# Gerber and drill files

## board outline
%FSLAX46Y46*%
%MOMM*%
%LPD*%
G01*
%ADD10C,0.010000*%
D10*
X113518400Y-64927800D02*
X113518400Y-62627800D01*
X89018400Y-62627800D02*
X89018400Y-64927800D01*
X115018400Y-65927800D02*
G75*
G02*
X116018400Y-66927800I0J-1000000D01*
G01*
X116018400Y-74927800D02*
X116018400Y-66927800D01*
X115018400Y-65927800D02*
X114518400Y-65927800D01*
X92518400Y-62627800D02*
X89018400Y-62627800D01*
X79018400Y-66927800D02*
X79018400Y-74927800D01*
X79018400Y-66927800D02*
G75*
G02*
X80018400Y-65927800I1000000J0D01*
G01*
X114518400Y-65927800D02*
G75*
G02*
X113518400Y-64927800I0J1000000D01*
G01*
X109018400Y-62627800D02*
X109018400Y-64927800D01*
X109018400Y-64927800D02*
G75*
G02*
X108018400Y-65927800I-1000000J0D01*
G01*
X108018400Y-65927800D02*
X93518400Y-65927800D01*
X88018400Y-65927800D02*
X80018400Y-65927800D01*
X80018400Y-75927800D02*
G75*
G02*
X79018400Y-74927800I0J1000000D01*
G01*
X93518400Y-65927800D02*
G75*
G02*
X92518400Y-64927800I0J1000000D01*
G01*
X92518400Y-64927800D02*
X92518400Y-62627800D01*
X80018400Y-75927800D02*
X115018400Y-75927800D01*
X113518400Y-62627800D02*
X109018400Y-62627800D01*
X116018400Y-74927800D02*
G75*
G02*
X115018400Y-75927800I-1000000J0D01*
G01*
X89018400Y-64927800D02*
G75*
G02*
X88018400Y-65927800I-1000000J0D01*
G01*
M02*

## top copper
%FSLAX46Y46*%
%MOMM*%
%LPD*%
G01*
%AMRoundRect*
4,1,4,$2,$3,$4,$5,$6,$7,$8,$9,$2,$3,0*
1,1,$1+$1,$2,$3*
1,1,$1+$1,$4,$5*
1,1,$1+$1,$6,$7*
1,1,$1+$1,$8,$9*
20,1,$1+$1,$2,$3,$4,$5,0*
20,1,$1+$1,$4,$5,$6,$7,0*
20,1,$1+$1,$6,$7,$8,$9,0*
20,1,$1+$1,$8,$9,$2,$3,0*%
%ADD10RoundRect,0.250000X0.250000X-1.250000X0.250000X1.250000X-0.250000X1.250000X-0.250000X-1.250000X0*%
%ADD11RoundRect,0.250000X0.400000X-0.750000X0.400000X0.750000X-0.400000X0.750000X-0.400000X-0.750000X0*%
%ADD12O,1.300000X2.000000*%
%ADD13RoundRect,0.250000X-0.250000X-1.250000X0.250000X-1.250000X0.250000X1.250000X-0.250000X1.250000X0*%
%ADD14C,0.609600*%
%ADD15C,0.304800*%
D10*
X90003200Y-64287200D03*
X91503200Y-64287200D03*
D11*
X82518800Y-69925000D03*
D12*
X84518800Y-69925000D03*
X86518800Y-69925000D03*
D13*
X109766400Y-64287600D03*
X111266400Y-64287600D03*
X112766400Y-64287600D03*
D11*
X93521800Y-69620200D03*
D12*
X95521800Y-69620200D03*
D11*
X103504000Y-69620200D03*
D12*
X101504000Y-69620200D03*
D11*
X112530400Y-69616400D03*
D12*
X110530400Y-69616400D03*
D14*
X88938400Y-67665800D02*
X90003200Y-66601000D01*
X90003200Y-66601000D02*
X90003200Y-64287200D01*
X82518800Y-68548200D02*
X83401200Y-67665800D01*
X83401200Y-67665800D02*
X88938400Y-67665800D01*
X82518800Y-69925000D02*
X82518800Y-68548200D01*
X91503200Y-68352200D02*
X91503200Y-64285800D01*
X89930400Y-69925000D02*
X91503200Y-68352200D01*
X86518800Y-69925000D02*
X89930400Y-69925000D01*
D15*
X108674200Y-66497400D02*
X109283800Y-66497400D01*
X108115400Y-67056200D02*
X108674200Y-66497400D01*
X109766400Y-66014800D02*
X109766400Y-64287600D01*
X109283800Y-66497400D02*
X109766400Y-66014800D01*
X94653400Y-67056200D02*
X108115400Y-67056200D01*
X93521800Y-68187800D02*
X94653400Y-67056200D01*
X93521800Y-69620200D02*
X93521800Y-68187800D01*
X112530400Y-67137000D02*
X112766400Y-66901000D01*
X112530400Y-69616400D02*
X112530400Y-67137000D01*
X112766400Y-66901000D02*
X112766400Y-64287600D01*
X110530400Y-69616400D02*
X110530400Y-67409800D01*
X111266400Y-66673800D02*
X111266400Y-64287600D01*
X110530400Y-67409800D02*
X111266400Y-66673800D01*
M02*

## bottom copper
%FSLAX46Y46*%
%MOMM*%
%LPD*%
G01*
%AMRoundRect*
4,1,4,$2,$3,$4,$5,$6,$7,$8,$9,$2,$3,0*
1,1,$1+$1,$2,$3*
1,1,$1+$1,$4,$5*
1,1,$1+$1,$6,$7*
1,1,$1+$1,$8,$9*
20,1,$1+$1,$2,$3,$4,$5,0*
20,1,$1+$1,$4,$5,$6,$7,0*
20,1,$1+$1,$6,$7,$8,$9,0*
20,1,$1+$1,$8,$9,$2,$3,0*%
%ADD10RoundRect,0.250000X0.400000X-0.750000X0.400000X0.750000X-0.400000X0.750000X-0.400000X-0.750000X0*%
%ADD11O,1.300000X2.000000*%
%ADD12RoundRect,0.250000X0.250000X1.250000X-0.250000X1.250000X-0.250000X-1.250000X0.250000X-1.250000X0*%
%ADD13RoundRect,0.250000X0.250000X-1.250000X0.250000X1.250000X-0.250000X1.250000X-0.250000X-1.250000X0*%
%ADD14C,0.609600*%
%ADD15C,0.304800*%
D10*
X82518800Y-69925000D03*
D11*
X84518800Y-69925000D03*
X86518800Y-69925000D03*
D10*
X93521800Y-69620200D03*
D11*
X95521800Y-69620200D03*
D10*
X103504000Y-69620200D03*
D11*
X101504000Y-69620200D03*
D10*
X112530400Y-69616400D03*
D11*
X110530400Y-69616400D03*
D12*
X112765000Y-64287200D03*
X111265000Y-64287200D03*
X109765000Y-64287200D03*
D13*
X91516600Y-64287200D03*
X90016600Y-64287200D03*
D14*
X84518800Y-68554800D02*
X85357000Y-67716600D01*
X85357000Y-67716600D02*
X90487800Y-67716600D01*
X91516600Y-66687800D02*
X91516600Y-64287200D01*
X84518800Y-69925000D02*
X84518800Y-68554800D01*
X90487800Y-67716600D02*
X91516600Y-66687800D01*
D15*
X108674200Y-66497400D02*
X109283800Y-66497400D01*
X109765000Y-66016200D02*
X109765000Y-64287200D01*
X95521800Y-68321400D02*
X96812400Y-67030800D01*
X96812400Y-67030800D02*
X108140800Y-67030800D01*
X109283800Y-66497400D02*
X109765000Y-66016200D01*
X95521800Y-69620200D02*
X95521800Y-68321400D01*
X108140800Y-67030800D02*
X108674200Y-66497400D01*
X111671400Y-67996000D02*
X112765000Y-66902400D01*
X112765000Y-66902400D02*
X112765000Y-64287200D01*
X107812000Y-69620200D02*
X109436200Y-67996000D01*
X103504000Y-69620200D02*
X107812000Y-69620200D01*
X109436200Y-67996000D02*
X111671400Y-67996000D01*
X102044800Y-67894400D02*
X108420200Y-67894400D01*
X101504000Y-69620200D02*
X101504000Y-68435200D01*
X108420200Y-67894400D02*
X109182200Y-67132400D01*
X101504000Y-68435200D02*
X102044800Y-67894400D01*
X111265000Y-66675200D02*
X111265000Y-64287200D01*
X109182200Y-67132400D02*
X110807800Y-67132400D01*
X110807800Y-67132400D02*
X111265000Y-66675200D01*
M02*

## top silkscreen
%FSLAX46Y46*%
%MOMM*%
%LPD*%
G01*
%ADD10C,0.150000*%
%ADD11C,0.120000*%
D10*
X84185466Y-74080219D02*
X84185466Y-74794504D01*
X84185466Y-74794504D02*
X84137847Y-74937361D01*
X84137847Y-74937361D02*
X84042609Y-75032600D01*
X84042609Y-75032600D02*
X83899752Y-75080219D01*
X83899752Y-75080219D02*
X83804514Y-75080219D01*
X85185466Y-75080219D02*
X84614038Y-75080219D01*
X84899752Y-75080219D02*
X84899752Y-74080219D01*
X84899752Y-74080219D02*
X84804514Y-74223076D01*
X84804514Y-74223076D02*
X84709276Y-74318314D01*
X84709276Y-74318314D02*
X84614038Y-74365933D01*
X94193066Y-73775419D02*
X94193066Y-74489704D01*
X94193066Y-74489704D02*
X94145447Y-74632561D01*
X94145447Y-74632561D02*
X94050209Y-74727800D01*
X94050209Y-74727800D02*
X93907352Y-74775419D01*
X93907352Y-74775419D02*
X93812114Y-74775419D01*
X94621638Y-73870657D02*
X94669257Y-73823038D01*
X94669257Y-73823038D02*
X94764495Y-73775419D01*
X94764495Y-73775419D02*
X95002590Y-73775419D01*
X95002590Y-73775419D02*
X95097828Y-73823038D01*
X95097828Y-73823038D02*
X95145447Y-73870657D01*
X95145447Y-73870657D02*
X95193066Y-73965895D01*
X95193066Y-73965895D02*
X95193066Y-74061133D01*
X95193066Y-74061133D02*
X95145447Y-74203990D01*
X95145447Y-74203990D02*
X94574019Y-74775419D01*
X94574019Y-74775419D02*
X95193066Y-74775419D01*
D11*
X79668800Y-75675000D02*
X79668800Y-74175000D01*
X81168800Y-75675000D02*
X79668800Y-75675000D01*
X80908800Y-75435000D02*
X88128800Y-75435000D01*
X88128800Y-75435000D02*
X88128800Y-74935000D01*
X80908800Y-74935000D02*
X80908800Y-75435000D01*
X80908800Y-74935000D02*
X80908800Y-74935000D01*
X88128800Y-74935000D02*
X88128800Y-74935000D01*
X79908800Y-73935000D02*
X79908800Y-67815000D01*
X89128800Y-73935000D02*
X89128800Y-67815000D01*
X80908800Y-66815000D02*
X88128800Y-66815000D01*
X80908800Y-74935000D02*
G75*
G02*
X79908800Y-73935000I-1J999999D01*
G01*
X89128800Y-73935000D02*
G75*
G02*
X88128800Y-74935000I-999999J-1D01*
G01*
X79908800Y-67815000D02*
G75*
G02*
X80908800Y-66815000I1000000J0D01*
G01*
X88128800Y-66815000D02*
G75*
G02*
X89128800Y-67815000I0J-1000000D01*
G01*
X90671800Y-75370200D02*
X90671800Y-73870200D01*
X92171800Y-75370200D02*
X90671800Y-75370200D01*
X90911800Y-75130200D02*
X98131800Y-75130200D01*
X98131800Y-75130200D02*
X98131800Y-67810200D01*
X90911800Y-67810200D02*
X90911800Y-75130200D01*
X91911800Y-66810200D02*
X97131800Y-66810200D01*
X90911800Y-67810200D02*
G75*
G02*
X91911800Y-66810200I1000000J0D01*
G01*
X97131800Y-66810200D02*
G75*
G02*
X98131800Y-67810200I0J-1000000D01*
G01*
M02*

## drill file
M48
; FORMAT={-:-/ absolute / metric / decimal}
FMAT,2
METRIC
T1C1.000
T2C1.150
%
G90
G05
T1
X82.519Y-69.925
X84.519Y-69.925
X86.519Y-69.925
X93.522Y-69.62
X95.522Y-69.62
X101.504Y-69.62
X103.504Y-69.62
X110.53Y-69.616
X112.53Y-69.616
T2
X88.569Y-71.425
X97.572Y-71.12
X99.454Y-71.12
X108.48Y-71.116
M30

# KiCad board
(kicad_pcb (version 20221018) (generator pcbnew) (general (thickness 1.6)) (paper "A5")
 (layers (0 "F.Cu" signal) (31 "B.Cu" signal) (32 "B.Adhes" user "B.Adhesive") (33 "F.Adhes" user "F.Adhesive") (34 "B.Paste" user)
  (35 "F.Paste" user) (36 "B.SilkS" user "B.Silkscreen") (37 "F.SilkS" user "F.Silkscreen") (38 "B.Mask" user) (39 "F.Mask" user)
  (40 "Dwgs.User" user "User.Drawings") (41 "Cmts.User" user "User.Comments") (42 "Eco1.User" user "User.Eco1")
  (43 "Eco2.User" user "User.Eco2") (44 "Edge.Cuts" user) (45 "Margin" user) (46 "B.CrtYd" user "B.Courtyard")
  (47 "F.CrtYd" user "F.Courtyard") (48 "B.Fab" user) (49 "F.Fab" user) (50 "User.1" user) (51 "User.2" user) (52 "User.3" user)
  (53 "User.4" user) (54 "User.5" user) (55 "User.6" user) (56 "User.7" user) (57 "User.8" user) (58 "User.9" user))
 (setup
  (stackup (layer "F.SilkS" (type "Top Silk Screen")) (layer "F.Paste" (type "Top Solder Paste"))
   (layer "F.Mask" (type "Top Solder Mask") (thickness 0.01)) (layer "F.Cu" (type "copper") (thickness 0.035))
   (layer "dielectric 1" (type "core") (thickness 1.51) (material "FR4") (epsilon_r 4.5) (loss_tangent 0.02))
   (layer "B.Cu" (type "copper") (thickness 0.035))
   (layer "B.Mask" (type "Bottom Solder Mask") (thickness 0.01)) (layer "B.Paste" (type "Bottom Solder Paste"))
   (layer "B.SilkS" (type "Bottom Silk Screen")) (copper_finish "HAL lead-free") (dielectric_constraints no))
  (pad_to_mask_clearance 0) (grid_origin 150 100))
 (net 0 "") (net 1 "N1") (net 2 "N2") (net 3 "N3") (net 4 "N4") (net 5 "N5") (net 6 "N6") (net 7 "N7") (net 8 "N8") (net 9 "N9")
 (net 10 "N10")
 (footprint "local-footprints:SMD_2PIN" (layer "F.Cu") (at 90.7532 63.7872)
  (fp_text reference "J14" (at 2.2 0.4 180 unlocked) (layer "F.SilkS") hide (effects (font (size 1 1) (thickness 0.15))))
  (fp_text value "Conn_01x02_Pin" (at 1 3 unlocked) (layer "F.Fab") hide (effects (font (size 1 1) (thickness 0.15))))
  (pad "1" smd roundrect (at -0.75 0.5 90) (size 3 1) (layers "F.Cu" "F.Paste" "F.Mask") (roundrect_rratio 0.25) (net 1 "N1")
   (thermal_bridge_angle 45))
  (pad "2" smd roundrect (at 0.75 0.5 90) (size 3 1) (layers "F.Cu" "F.Paste" "F.Mask") (roundrect_rratio 0.25) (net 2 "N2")
   (thermal_bridge_angle 45)))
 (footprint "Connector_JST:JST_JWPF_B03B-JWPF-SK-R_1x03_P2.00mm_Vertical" (layer "F.Cu") (at 82.5188 69.925 90)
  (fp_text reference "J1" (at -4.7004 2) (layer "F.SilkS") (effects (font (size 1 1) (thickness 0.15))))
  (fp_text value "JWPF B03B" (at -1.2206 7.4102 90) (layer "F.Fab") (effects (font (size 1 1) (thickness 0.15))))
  (fp_line (start -5.75 -2.85) (end -4.25 -2.85) (stroke (width 0.12) (type solid)) (layer "F.SilkS"))
  (fp_line (start -5.75 -1.35) (end -5.75 -2.85) (stroke (width 0.12) (type solid)) (layer "F.SilkS"))
  (fp_line (start -5.51 -1.61) (end -5.51 5.61) (stroke (width 0.12) (type solid)) (layer "F.SilkS"))
  (fp_line (start -5.51 5.61) (end -5.01 5.61) (stroke (width 0.12) (type solid)) (layer "F.SilkS"))
  (fp_line (start -5.01 -1.61) (end -5.51 -1.61) (stroke (width 0.12) (type solid)) (layer "F.SilkS"))
  (fp_line (start -5.01 -1.61) (end -5.01 -1.61) (stroke (width 0.12) (type solid)) (layer "F.SilkS"))
  (fp_line (start -5.01 5.61) (end -5.01 5.61) (stroke (width 0.12) (type solid)) (layer "F.SilkS"))
  (fp_line (start -4.01 -2.61) (end 2.11 -2.61) (stroke (width 0.12) (type solid)) (layer "F.SilkS"))
  (fp_line (start -4.01 6.61) (end 2.11 6.61) (stroke (width 0.12) (type solid)) (layer "F.SilkS"))
  (fp_line (start 3.11 -1.61) (end 3.11 5.61) (stroke (width 0.12) (type solid)) (layer "F.SilkS"))
  (fp_arc (start -5.01 -1.61) (mid -4.717107 -2.317107) (end -4.01 -2.61) (stroke (width 0.12) (type solid)) (layer "F.SilkS"))
  (fp_arc (start -4.01 6.61) (mid -4.717107 6.317107) (end -5.01 5.61) (stroke (width 0.12) (type solid)) (layer "F.SilkS"))
  (fp_arc (start 2.11 -2.61) (mid 2.817107 -2.317107) (end 3.11 -1.61) (stroke (width 0.12) (type solid)) (layer "F.SilkS"))
  (fp_arc (start 3.11 5.61) (mid 2.817107 6.317107) (end 2.11 6.61) (stroke (width 0.12) (type solid)) (layer "F.SilkS"))
  (pad "" np_thru_hole circle (at -1.5 6.05 90) (size 1.15 1.15) (drill 1.15) (layers "*.Cu" "*.Mask"))
  (pad "1" thru_hole roundrect (at 0 0 90) (size 2 1.3) (drill 1) (layers "*.Cu" "*.Mask") (roundrect_rratio 0.1923076923) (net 1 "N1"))
  (pad "2" thru_hole oval (at 0 2 90) (size 2 1.3) (drill 1) (layers "*.Cu" "*.Mask") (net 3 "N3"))
  (pad "3" thru_hole oval (at 0 4 90) (size 2 1.3) (drill 1) (layers "*.Cu" "*.Mask") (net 2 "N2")))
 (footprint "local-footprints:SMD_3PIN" (layer "F.Cu") (at 111.2664 63.7876)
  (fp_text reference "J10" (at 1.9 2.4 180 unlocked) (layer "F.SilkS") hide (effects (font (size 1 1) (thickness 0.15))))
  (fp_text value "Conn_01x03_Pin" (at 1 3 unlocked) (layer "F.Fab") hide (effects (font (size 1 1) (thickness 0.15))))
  (pad "1" smd roundrect (at -1.5 0.5) (size 1 3) (layers "F.Cu" "F.Paste" "F.Mask") (roundrect_rratio 0.25) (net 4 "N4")
   (thermal_bridge_angle 45))
  (pad "2" smd roundrect (at 0 0.5) (size 1 3) (layers "F.Cu" "F.Paste" "F.Mask") (roundrect_rratio 0.25) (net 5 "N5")
   (thermal_bridge_angle 45))
  (pad "3" smd roundrect (at 1.5 0.5) (size 1 3) (layers "F.Cu" "F.Paste" "F.Mask") (roundrect_rratio 0.25) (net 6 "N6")
   (thermal_bridge_angle 45)))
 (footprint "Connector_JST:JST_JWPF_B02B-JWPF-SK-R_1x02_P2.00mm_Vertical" (layer "F.Cu") (at 93.5218 69.6202 90)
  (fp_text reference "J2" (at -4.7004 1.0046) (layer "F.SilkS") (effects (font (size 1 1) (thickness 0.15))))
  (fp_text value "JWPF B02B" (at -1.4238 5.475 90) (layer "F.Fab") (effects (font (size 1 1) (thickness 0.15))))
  (fp_line (start -5.75 -2.85) (end -4.25 -2.85) (stroke (width 0.12) (type solid)) (layer "F.SilkS"))
  (fp_line (start -5.75 -1.35) (end -5.75 -2.85) (stroke (width 0.12) (type solid)) (layer "F.SilkS"))
  (fp_line (start -5.51 -2.61) (end -5.51 4.61) (stroke (width 0.12) (type solid)) (layer "F.SilkS"))
  (fp_line (start -5.51 4.61) (end 1.81 4.61) (stroke (width 0.12) (type solid)) (layer "F.SilkS"))
  (fp_line (start 1.81 -2.61) (end -5.51 -2.61) (stroke (width 0.12) (type solid)) (layer "F.SilkS"))
  (fp_line (start 2.81 -1.61) (end 2.81 3.61) (stroke (width 0.12) (type solid)) (layer "F.SilkS"))
  (fp_arc (start 1.81 -2.61) (mid 2.517107 -2.317107) (end 2.81 -1.61) (stroke (width 0.12) (type solid)) (layer "F.SilkS"))
  (fp_arc (start 2.81 3.61) (mid 2.517107 4.317107) (end 1.81 4.61) (stroke (width 0.12) (type solid)) (layer "F.SilkS"))
  (pad "" np_thru_hole circle (at -1.5 4.05 90) (size 1.15 1.15) (drill 1.15) (layers "*.Cu" "*.Mask"))
  (pad "1" thru_hole roundrect (at 0 0 90) (size 2 1.3) (drill 1) (layers "*.Cu" "*.Mask") (roundrect_rratio 0.1923076923) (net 4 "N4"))
  (pad "2" thru_hole oval (at 0 2 90) (size 2 1.3) (drill 1) (layers "*.Cu" "*.Mask") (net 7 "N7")))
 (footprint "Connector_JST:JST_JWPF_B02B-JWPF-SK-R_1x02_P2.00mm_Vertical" (layer "B.Cu") (at 103.504 69.6202 90)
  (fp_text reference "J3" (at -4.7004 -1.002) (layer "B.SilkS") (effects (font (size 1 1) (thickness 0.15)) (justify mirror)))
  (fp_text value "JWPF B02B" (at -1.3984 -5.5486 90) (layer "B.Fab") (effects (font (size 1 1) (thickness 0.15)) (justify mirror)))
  (pad "" np_thru_hole circle (at -1.5 -4.05 90) (size 1.15 1.15) (drill 1.15) (layers "*.Cu" "*.Mask"))
  (pad "1" thru_hole roundrect (at 0 0 90) (size 2 1.3) (drill 1) (layers "*.Cu" "*.Mask") (roundrect_rratio 0.1923076923) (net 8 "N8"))
  (pad "2" thru_hole oval (at 0 -2 90) (size 2 1.3) (drill 1) (layers "*.Cu" "*.Mask") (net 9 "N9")))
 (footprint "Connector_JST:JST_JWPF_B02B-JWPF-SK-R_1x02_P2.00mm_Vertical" (layer "B.Cu") (at 112.5304 69.6164 90)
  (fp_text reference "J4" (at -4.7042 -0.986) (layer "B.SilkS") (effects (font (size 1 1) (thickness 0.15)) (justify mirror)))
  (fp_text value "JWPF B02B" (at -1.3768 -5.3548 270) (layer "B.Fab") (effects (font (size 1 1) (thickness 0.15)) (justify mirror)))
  (pad "" np_thru_hole circle (at -1.5 -4.05 90) (size 1.15 1.15) (drill 1.15) (layers "*.Cu" "*.Mask"))
  (pad "1" thru_hole roundrect (at 0 0 90) (size 2 1.3) (drill 1) (layers "*.Cu" "*.Mask") (roundrect_rratio 0.1923076923) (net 6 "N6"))
  (pad "2" thru_hole oval (at 0 -2 90) (size 2 1.3) (drill 1) (layers "*.Cu" "*.Mask") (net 5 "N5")))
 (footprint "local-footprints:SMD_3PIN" (layer "B.Cu") (at 111.265 63.7872 180)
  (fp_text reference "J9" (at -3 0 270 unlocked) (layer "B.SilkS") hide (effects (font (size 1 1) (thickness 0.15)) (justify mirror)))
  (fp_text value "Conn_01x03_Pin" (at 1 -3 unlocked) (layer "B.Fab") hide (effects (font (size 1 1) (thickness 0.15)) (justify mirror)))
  (pad "1" smd roundrect (at -1.5 -0.5 180) (size 1 3) (layers "B.Cu" "B.Paste" "B.Mask") (roundrect_rratio 0.25) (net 8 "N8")
   (thermal_bridge_angle 45))
  (pad "2" smd roundrect (at 0 -0.5 180) (size 1 3) (layers "B.Cu" "B.Paste" "B.Mask") (roundrect_rratio 0.25) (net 9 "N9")
   (thermal_bridge_angle 45))
  (pad "3" smd roundrect (at 1.5 -0.5 180) (size 1 3) (layers "B.Cu" "B.Paste" "B.Mask") (roundrect_rratio 0.25) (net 7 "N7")
   (thermal_bridge_angle 45)))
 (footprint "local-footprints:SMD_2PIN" (layer "B.Cu") (at 90.7666 63.7872 180)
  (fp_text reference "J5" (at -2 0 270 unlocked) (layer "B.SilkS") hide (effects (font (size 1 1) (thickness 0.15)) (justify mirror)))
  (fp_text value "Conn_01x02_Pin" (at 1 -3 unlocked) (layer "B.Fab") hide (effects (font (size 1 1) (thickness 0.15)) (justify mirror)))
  (pad "1" smd roundrect (at -0.75 -0.5 90) (size 3 1) (layers "B.Cu" "B.Paste" "B.Mask") (roundrect_rratio 0.25) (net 3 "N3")
   (thermal_bridge_angle 45))
  (pad "2" smd roundrect (at 0.75 -0.5 90) (size 3 1) (layers "B.Cu" "B.Paste" "B.Mask") (roundrect_rratio 0.25) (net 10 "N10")
   (thermal_bridge_angle 45)))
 (gr_line (start 113.5184 64.9278) (end 113.5184 62.6278) (stroke (width 0.01) (type solid)) (layer "Edge.Cuts"))
 (gr_line (start 89.0184 62.6278) (end 89.0184 64.9278) (stroke (width 0.01) (type solid)) (layer "Edge.Cuts"))
 (gr_arc (start 115.0184 65.9278) (mid 115.725507 66.220693) (end 116.0184 66.9278) (stroke (width 0.01) (type solid)) (layer "Edge.Cuts"))
 (gr_line (start 116.0184 74.9278) (end 116.0184 66.9278) (stroke (width 0.01) (type solid)) (layer "Edge.Cuts"))
 (gr_line (start 115.0184 65.9278) (end 114.5184 65.9278) (stroke (width 0.01) (type solid)) (layer "Edge.Cuts"))
 (gr_line (start 92.5184 62.6278) (end 89.0184 62.6278) (stroke (width 0.01) (type solid)) (layer "Edge.Cuts"))
 (gr_line (start 79.0184 66.9278) (end 79.0184 74.9278) (stroke (width 0.01) (type solid)) (layer "Edge.Cuts"))
 (gr_arc (start 79.0184 66.9278) (mid 79.311293 66.220693) (end 80.0184 65.9278) (stroke (width 0.01) (type solid)) (layer "Edge.Cuts"))
 (gr_arc (start 114.5184 65.9278) (mid 113.811293 65.634907) (end 113.5184 64.9278) (stroke (width 0.01) (type solid)) (layer "Edge.Cuts"))
 (gr_line (start 109.0184 62.6278) (end 109.0184 64.9278) (stroke (width 0.01) (type solid)) (layer "Edge.Cuts"))
 (gr_arc (start 109.0184 64.9278) (mid 108.725507 65.634907) (end 108.0184 65.9278) (stroke (width 0.01) (type solid)) (layer "Edge.Cuts"))
 (gr_line (start 108.0184 65.9278) (end 93.5184 65.9278) (stroke (width 0.01) (type solid)) (layer "Edge.Cuts"))
 (gr_line (start 88.0184 65.9278) (end 80.0184 65.9278) (stroke (width 0.01) (type solid)) (layer "Edge.Cuts"))
 (gr_arc (start 80.0184 75.9278) (mid 79.311293 75.634907) (end 79.0184 74.9278) (stroke (width 0.01) (type solid)) (layer "Edge.Cuts"))
 (gr_arc (start 93.5184 65.9278) (mid 92.811293 65.634907) (end 92.5184 64.9278) (stroke (width 0.01) (type solid)) (layer "Edge.Cuts"))
 (gr_line (start 92.5184 64.9278) (end 92.5184 62.6278) (stroke (width 0.01) (type solid)) (layer "Edge.Cuts"))
 (gr_line (start 80.0184 75.9278) (end 115.0184 75.9278) (stroke (width 0.01) (type solid)) (layer "Edge.Cuts"))
 (gr_line (start 113.5184 62.6278) (end 109.0184 62.6278) (stroke (width 0.01) (type solid)) (layer "Edge.Cuts"))
 (gr_arc (start 116.0184 74.9278) (mid 115.725507 75.634907) (end 115.0184 75.9278) (stroke (width 0.01) (type solid)) (layer "Edge.Cuts"))
 (gr_arc (start 89.0184 64.9278) (mid 88.725507 65.634907) (end 88.0184 65.9278) (stroke (width 0.01) (type solid)) (layer "Edge.Cuts"))
 (segment (start 88.9384 67.6658) (end 90.0032 66.601) (width 0.6096) (layer "F.Cu") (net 1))
 (segment (start 90.0032 66.601) (end 90.0032 64.2872) (width 0.6096) (layer "F.Cu") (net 1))
 (segment (start 82.5188 68.5482) (end 83.4012 67.6658) (width 0.6096) (layer "F.Cu") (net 1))
 (segment (start 83.4012 67.6658) (end 88.9384 67.6658) (width 0.6096) (layer "F.Cu") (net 1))
 (segment (start 82.5188 69.925) (end 82.5188 68.5482) (width 0.6096) (layer "F.Cu") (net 1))
 (segment (start 84.5188 68.5548) (end 85.357 67.7166) (width 0.6096) (layer "B.Cu") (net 3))
 (segment (start 85.357 67.7166) (end 90.4878 67.7166) (width 0.6096) (layer "B.Cu") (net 3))
 (segment (start 91.5166 66.6878) (end 91.5166 64.2872) (width 0.6096) (layer "B.Cu") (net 3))
 (segment (start 84.5188 69.925) (end 84.5188 68.5548) (width 0.6096) (layer "B.Cu") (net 3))
 (segment (start 90.4878 67.7166) (end 91.5166 66.6878) (width 0.6096) (layer "B.Cu") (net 3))
 (segment (start 91.5032 68.3522) (end 91.5032 64.2858) (width 0.6096) (layer "F.Cu") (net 2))
 (segment (start 89.9304 69.925) (end 91.5032 68.3522) (width 0.6096) (layer "F.Cu") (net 2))
 (segment (start 86.5188 69.925) (end 89.9304 69.925) (width 0.6096) (layer "F.Cu") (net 2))
 (segment (start 108.6742 66.4974) (end 109.2838 66.4974) (width 0.3048) (layer "F.Cu") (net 4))
 (segment (start 108.1154 67.0562) (end 108.6742 66.4974) (width 0.3048) (layer "F.Cu") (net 4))
 (segment (start 109.7664 66.0148) (end 109.7664 64.2876) (width 0.3048) (layer "F.Cu") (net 4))
 (segment (start 109.2838 66.4974) (end 109.7664 66.0148) (width 0.3048) (layer "F.Cu") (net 4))
 (segment (start 94.6534 67.0562) (end 108.1154 67.0562) (width 0.3048) (layer "F.Cu") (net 4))
 (segment (start 93.5218 68.1878) (end 94.6534 67.0562) (width 0.3048) (layer "F.Cu") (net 4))
 (segment (start 93.5218 69.6202) (end 93.5218 68.1878) (width 0.3048) (layer "F.Cu") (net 4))
 (segment (start 108.6742 66.4974) (end 109.2838 66.4974) (width 0.3048) (layer "B.Cu") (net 7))
 (segment (start 109.765 66.0162) (end 109.765 64.2872) (width 0.3048) (layer "B.Cu") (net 7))
 (segment (start 95.5218 68.3214) (end 96.8124 67.0308) (width 0.3048) (layer "B.Cu") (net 7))
 (segment (start 96.8124 67.0308) (end 108.1408 67.0308) (width 0.3048) (layer "B.Cu") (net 7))
 (segment (start 109.2838 66.4974) (end 109.765 66.0162) (width 0.3048) (layer "B.Cu") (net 7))
 (segment (start 95.5218 69.6202) (end 95.5218 68.3214) (width 0.3048) (layer "B.Cu") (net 7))
 (segment (start 108.1408 67.0308) (end 108.6742 66.4974) (width 0.3048) (layer "B.Cu") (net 7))
 (segment (start 111.6714 67.996) (end 112.765 66.9024) (width 0.3048) (layer "B.Cu") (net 8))
 (segment (start 112.765 66.9024) (end 112.765 64.2872) (width 0.3048) (layer "B.Cu") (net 8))
 (segment (start 107.812 69.6202) (end 109.4362 67.996) (width 0.3048) (layer "B.Cu") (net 8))
 (segment (start 103.504 69.6202) (end 107.812 69.6202) (width 0.3048) (layer "B.Cu") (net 8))
 (segment (start 109.4362 67.996) (end 111.6714 67.996) (width 0.3048) (layer "B.Cu") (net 8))
 (segment (start 102.0448 67.8944) (end 108.4202 67.8944) (width 0.3048) (layer "B.Cu") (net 9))
 (segment (start 101.504 69.6202) (end 101.504 68.4352) (width 0.3048) (layer "B.Cu") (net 9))
 (segment (start 108.4202 67.8944) (end 109.1822 67.1324) (width 0.3048) (layer "B.Cu") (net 9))
 (segment (start 101.504 68.4352) (end 102.0448 67.8944) (width 0.3048) (layer "B.Cu") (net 9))
 (segment (start 111.265 66.6752) (end 111.265 64.2872) (width 0.3048) (layer "B.Cu") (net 9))
 (segment (start 109.1822 67.1324) (end 110.8078 67.1324) (width 0.3048) (layer "B.Cu") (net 9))
 (segment (start 110.8078 67.1324) (end 111.265 66.6752) (width 0.3048) (layer "B.Cu") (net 9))
 (segment (start 112.5304 67.137) (end 112.7664 66.901) (width 0.3048) (layer "F.Cu") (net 6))
 (segment (start 112.5304 69.6164) (end 112.5304 67.137) (width 0.3048) (layer "F.Cu") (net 6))
 (segment (start 112.7664 66.901) (end 112.7664 64.2876) (width 0.3048) (layer "F.Cu") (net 6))
 (segment (start 110.5304 69.6164) (end 110.5304 67.4098) (width 0.3048) (layer "F.Cu") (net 5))
 (segment (start 111.2664 66.6738) (end 111.2664 64.2876) (width 0.3048) (layer "F.Cu") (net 5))
 (segment (start 110.5304 67.4098) (end 111.2664 66.6738) (width 0.3048) (layer "F.Cu") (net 5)))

